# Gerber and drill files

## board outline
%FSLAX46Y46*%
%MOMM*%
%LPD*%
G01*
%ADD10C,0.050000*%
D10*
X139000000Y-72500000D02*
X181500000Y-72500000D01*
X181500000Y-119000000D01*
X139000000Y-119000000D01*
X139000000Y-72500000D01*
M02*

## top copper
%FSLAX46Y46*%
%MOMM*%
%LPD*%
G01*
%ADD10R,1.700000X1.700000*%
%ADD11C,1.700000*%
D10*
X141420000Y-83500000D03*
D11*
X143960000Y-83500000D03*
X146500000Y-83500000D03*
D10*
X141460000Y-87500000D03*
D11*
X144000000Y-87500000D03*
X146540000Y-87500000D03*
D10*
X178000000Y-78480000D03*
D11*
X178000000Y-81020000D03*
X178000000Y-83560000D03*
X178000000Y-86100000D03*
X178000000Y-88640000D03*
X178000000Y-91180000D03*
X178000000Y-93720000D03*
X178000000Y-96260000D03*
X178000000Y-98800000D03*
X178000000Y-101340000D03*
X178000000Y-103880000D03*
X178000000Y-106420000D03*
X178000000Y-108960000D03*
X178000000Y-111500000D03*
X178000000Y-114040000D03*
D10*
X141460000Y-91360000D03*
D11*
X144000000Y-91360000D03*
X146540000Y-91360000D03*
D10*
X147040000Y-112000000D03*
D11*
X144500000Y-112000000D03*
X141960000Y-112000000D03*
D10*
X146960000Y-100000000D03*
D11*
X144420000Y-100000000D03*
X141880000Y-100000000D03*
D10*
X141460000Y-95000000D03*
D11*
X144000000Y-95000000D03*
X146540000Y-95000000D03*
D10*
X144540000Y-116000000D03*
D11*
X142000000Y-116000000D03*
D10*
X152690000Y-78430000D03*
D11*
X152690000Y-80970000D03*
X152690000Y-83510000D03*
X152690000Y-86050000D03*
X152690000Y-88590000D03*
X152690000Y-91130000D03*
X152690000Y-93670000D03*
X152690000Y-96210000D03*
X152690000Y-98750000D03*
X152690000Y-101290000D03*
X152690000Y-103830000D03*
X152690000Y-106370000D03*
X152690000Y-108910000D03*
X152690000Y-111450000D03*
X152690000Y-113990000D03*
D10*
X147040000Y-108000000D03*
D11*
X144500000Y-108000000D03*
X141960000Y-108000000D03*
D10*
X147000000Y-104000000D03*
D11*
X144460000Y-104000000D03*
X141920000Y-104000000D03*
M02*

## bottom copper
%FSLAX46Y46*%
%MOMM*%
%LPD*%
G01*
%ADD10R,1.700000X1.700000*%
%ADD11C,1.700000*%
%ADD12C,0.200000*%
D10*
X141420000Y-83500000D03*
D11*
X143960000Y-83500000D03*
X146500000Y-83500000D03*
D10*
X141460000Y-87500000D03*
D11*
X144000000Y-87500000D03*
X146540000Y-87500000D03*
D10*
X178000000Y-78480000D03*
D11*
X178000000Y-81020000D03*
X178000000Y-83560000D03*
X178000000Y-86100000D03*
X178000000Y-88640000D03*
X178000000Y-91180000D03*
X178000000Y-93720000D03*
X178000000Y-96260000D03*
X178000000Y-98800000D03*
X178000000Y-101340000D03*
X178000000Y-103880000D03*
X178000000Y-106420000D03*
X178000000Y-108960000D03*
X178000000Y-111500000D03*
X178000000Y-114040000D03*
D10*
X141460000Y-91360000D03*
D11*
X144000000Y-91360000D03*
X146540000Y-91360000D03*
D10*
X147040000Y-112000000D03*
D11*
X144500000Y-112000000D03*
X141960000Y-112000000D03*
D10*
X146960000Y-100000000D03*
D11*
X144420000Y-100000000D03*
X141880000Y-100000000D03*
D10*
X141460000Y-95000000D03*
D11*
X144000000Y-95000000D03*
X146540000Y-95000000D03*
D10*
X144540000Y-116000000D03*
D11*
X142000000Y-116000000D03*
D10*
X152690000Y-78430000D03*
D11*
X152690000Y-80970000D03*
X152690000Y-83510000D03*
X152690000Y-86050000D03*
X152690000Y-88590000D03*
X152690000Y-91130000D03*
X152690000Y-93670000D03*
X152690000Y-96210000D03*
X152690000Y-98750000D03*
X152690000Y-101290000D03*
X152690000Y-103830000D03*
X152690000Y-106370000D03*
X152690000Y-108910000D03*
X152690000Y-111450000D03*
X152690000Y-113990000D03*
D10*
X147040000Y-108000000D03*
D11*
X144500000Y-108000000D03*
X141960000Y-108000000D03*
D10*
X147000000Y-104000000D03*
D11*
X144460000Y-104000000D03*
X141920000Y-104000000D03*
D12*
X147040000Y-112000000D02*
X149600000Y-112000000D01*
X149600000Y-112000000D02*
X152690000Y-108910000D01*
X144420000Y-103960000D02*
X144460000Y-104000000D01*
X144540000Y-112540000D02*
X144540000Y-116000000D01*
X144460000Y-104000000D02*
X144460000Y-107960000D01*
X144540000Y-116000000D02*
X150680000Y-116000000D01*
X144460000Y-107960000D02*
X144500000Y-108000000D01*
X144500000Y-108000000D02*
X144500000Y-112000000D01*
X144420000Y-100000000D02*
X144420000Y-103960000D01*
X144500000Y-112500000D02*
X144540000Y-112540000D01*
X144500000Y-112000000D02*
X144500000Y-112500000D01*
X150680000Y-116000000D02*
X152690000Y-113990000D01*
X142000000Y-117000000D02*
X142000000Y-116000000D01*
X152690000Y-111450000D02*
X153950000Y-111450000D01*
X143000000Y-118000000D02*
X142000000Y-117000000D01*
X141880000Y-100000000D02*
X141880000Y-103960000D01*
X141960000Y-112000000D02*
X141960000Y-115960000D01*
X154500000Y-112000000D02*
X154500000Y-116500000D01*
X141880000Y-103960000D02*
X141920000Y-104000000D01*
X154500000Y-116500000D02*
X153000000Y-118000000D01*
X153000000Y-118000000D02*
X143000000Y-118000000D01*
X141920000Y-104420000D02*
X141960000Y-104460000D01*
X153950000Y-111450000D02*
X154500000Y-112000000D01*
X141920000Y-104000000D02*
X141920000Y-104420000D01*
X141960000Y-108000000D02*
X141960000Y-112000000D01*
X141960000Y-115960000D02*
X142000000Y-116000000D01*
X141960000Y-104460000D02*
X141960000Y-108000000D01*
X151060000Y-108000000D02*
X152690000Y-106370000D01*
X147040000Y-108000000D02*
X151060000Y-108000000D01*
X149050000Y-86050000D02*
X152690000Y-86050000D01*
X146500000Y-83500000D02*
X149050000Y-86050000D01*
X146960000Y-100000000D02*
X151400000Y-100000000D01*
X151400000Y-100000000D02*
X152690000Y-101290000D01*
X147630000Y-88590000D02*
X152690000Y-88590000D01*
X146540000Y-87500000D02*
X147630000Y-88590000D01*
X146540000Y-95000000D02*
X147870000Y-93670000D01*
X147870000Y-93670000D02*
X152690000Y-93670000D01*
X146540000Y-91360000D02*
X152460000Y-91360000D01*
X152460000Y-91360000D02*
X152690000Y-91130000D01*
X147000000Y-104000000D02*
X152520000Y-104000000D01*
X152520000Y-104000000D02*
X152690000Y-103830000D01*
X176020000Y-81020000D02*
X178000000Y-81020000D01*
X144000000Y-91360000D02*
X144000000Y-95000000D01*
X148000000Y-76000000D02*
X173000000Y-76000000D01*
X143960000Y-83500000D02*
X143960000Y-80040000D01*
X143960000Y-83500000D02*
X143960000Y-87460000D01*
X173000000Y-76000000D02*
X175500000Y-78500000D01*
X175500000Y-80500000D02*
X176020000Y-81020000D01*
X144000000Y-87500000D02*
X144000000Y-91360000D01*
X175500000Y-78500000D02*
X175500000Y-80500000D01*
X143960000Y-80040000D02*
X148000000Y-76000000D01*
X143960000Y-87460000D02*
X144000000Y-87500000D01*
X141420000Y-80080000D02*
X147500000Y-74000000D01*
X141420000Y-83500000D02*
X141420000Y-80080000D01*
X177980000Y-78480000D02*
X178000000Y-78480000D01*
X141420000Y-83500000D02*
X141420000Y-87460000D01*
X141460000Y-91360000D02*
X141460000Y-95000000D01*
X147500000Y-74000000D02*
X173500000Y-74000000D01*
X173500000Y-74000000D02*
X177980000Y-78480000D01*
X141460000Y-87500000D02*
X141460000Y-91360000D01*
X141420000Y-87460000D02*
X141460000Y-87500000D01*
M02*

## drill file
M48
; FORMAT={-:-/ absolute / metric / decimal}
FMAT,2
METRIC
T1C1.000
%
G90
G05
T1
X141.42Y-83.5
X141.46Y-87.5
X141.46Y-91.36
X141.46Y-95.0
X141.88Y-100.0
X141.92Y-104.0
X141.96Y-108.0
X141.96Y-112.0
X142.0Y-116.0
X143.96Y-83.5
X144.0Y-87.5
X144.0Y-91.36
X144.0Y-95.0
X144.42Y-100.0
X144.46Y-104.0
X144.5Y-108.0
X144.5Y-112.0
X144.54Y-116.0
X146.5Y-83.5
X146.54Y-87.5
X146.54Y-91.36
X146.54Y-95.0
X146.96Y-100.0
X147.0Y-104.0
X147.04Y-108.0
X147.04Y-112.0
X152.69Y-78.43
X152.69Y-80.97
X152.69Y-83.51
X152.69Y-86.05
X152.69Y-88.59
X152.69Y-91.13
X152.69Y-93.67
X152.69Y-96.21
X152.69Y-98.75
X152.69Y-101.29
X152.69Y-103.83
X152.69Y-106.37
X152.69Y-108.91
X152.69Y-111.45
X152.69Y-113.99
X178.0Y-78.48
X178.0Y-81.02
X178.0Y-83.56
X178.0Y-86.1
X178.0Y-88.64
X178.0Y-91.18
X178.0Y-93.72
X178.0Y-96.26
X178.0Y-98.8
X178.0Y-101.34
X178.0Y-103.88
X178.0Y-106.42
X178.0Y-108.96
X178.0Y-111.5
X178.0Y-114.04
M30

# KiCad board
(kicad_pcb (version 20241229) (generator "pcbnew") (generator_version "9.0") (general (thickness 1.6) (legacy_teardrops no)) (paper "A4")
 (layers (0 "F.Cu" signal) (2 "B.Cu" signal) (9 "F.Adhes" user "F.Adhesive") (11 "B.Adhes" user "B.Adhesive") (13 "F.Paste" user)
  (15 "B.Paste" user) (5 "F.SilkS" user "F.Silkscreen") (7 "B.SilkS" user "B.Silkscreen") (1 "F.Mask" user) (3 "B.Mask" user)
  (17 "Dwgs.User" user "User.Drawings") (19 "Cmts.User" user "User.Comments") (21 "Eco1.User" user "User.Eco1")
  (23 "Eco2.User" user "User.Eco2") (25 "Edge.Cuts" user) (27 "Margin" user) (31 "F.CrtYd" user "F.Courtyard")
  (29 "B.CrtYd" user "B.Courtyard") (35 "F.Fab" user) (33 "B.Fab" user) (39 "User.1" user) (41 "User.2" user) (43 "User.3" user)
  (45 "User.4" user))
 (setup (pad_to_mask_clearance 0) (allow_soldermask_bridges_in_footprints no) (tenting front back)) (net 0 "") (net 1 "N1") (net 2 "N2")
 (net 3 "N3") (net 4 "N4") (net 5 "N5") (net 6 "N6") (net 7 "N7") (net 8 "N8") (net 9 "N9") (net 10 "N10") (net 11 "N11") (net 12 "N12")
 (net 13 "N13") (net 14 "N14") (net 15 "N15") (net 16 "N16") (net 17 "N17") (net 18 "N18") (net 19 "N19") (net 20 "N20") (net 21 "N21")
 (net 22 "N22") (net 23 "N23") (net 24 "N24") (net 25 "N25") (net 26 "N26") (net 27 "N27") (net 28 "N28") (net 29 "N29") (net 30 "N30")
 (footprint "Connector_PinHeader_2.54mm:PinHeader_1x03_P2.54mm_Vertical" (layer "F.Cu") (at 141.42 83.5 90)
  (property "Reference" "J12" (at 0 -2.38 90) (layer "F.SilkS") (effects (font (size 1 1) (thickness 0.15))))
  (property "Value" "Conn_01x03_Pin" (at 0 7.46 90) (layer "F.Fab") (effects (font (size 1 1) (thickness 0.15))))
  (pad "1" thru_hole rect (at 0 0 90) (size 1.7 1.7) (drill 1) (layers "*.Cu" "*.Mask") (remove_unused_layers no) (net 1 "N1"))
  (pad "2" thru_hole circle (at 0 2.54 90) (size 1.7 1.7) (drill 1) (layers "*.Cu" "*.Mask") (remove_unused_layers no) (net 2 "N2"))
  (pad "3" thru_hole circle (at 0 5.08 90) (size 1.7 1.7) (drill 1) (layers "*.Cu" "*.Mask") (remove_unused_layers no) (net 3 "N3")))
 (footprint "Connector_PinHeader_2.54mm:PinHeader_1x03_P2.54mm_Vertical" (layer "F.Cu") (at 141.46 87.5 90)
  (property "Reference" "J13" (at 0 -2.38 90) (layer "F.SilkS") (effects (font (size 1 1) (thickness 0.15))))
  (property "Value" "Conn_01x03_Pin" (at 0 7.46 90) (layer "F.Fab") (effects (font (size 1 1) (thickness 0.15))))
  (pad "1" thru_hole rect (at 0 0 90) (size 1.7 1.7) (drill 1) (layers "*.Cu" "*.Mask") (remove_unused_layers no) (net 1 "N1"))
  (pad "2" thru_hole circle (at 0 2.54 90) (size 1.7 1.7) (drill 1) (layers "*.Cu" "*.Mask") (remove_unused_layers no) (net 2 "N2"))
  (pad "3" thru_hole circle (at 0 5.08 90) (size 1.7 1.7) (drill 1) (layers "*.Cu" "*.Mask") (remove_unused_layers no) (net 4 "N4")))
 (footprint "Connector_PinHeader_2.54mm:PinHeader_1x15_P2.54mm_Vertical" (layer "F.Cu") (at 178 78.48)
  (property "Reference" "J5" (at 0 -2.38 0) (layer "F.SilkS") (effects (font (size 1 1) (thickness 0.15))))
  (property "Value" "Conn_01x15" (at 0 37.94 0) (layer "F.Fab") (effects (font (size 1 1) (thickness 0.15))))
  (pad "1" thru_hole rect (at 0 0) (size 1.7 1.7) (drill 1) (layers "*.Cu" "*.Mask") (remove_unused_layers no) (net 1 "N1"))
  (pad "2" thru_hole circle (at 0 2.54) (size 1.7 1.7) (drill 1) (layers "*.Cu" "*.Mask") (remove_unused_layers no) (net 2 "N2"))
  (pad "3" thru_hole circle (at 0 5.08) (size 1.7 1.7) (drill 1) (layers "*.Cu" "*.Mask") (remove_unused_layers no) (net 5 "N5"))
  (pad "4" thru_hole circle (at 0 7.62) (size 1.7 1.7) (drill 1) (layers "*.Cu" "*.Mask") (remove_unused_layers no) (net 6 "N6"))
  (pad "5" thru_hole circle (at 0 10.16) (size 1.7 1.7) (drill 1) (layers "*.Cu" "*.Mask") (remove_unused_layers no) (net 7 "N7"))
  (pad "6" thru_hole circle (at 0 12.7) (size 1.7 1.7) (drill 1) (layers "*.Cu" "*.Mask") (remove_unused_layers no) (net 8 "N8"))
  (pad "7" thru_hole circle (at 0 15.24) (size 1.7 1.7) (drill 1) (layers "*.Cu" "*.Mask") (remove_unused_layers no) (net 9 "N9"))
  (pad "8" thru_hole circle (at 0 17.78) (size 1.7 1.7) (drill 1) (layers "*.Cu" "*.Mask") (remove_unused_layers no) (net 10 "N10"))
  (pad "9" thru_hole circle (at 0 20.32) (size 1.7 1.7) (drill 1) (layers "*.Cu" "*.Mask") (remove_unused_layers no) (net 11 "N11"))
  (pad "10" thru_hole circle (at 0 22.86) (size 1.7 1.7) (drill 1) (layers "*.Cu" "*.Mask") (remove_unused_layers no) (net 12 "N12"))
  (pad "11" thru_hole circle (at 0 25.4) (size 1.7 1.7) (drill 1) (layers "*.Cu" "*.Mask") (remove_unused_layers no) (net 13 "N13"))
  (pad "12" thru_hole circle (at 0 27.94) (size 1.7 1.7) (drill 1) (layers "*.Cu" "*.Mask") (remove_unused_layers no) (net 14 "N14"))
  (pad "13" thru_hole circle (at 0 30.48) (size 1.7 1.7) (drill 1) (layers "*.Cu" "*.Mask") (remove_unused_layers no) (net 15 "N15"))
  (pad "14" thru_hole circle (at 0 33.02) (size 1.7 1.7) (drill 1) (layers "*.Cu" "*.Mask") (remove_unused_layers no) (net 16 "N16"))
  (pad "15" thru_hole circle (at 0 35.56) (size 1.7 1.7) (drill 1) (layers "*.Cu" "*.Mask") (remove_unused_layers no) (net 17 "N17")))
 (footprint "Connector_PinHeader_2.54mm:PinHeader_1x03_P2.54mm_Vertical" (layer "F.Cu") (at 141.46 91.36 90)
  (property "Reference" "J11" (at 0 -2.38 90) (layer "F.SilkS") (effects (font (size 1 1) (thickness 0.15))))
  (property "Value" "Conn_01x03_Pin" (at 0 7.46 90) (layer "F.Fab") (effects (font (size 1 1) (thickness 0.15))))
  (pad "1" thru_hole rect (at 0 0 90) (size 1.7 1.7) (drill 1) (layers "*.Cu" "*.Mask") (remove_unused_layers no) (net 1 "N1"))
  (pad "2" thru_hole circle (at 0 2.54 90) (size 1.7 1.7) (drill 1) (layers "*.Cu" "*.Mask") (remove_unused_layers no) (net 2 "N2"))
  (pad "3" thru_hole circle (at 0 5.08 90) (size 1.7 1.7) (drill 1) (layers "*.Cu" "*.Mask") (remove_unused_layers no) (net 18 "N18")))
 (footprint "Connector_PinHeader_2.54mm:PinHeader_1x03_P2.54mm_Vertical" (layer "F.Cu") (at 147.04 112 -90)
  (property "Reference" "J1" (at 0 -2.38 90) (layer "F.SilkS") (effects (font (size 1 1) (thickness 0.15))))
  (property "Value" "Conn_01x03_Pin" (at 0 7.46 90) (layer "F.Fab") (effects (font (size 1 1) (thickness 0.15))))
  (pad "1" thru_hole rect (at 0 0 270) (size 1.7 1.7) (drill 1) (layers "*.Cu" "*.Mask") (remove_unused_layers no) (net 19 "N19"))
  (pad "2" thru_hole circle (at 0 2.54 270) (size 1.7 1.7) (drill 1) (layers "*.Cu" "*.Mask") (remove_unused_layers no) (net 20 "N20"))
  (pad "3" thru_hole circle (at 0 5.08 270) (size 1.7 1.7) (drill 1) (layers "*.Cu" "*.Mask") (remove_unused_layers no) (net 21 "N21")))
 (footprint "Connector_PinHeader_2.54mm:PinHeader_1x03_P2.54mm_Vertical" (layer "F.Cu") (at 146.96 100 -90)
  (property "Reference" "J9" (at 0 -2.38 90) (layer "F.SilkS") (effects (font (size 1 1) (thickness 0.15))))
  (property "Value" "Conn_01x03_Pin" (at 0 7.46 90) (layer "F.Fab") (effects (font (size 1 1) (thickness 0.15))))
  (pad "1" thru_hole rect (at 0 0 270) (size 1.7 1.7) (drill 1) (layers "*.Cu" "*.Mask") (remove_unused_layers no) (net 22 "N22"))
  (pad "2" thru_hole circle (at 0 2.54 270) (size 1.7 1.7) (drill 1) (layers "*.Cu" "*.Mask") (remove_unused_layers no) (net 20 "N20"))
  (pad "3" thru_hole circle (at 0 5.08 270) (size 1.7 1.7) (drill 1) (layers "*.Cu" "*.Mask") (remove_unused_layers no) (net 21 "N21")))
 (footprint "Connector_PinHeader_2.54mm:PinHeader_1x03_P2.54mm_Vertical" (layer "F.Cu") (at 141.46 95 90)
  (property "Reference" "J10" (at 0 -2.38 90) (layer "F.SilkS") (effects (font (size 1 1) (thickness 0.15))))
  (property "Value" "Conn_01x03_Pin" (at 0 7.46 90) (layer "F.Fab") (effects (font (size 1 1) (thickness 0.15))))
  (pad "1" thru_hole rect (at 0 0 90) (size 1.7 1.7) (drill 1) (layers "*.Cu" "*.Mask") (remove_unused_layers no) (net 1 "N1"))
  (pad "2" thru_hole circle (at 0 2.54 90) (size 1.7 1.7) (drill 1) (layers "*.Cu" "*.Mask") (remove_unused_layers no) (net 2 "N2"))
  (pad "3" thru_hole circle (at 0 5.08 90) (size 1.7 1.7) (drill 1) (layers "*.Cu" "*.Mask") (remove_unused_layers no) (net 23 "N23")))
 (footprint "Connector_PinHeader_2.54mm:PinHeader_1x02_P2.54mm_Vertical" (layer "F.Cu") (at 144.54 116 -90)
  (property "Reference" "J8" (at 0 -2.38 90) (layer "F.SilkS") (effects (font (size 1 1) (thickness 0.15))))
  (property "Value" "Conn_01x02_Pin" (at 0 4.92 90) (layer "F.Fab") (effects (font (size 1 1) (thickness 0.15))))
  (pad "1" thru_hole rect (at 0 0 270) (size 1.7 1.7) (drill 1) (layers "*.Cu" "*.Mask") (remove_unused_layers no) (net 20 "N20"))
  (pad "2" thru_hole circle (at 0 2.54 270) (size 1.7 1.7) (drill 1) (layers "*.Cu" "*.Mask") (remove_unused_layers no) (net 21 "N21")))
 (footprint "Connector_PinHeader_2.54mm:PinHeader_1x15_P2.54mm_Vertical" (layer "F.Cu") (at 152.69 78.43)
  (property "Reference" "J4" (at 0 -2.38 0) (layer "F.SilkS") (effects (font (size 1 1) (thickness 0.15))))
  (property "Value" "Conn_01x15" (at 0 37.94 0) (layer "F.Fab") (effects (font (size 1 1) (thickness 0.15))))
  (pad "1" thru_hole rect (at 0 0) (size 1.7 1.7) (drill 1) (layers "*.Cu" "*.Mask") (remove_unused_layers no) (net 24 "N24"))
  (pad "2" thru_hole circle (at 0 2.54) (size 1.7 1.7) (drill 1) (layers "*.Cu" "*.Mask") (remove_unused_layers no) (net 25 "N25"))
  (pad "3" thru_hole circle (at 0 5.08) (size 1.7 1.7) (drill 1) (layers "*.Cu" "*.Mask") (remove_unused_layers no) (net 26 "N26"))
  (pad "4" thru_hole circle (at 0 7.62) (size 1.7 1.7) (drill 1) (layers "*.Cu" "*.Mask") (remove_unused_layers no) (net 3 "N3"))
  (pad "5" thru_hole circle (at 0 10.16) (size 1.7 1.7) (drill 1) (layers "*.Cu" "*.Mask") (remove_unused_layers no) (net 4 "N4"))
  (pad "6" thru_hole circle (at 0 12.7) (size 1.7 1.7) (drill 1) (layers "*.Cu" "*.Mask") (remove_unused_layers no) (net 18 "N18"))
  (pad "7" thru_hole circle (at 0 15.24) (size 1.7 1.7) (drill 1) (layers "*.Cu" "*.Mask") (remove_unused_layers no) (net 23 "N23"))
  (pad "8" thru_hole circle (at 0 17.78) (size 1.7 1.7) (drill 1) (layers "*.Cu" "*.Mask") (remove_unused_layers no) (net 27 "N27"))
  (pad "9" thru_hole circle (at 0 20.32) (size 1.7 1.7) (drill 1) (layers "*.Cu" "*.Mask") (remove_unused_layers no) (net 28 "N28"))
  (pad "10" thru_hole circle (at 0 22.86) (size 1.7 1.7) (drill 1) (layers "*.Cu" "*.Mask") (remove_unused_layers no) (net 22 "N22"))
  (pad "11" thru_hole circle (at 0 25.4) (size 1.7 1.7) (drill 1) (layers "*.Cu" "*.Mask") (remove_unused_layers no) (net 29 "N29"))
  (pad "12" thru_hole circle (at 0 27.94) (size 1.7 1.7) (drill 1) (layers "*.Cu" "*.Mask") (remove_unused_layers no) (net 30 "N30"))
  (pad "13" thru_hole circle (at 0 30.48) (size 1.7 1.7) (drill 1) (layers "*.Cu" "*.Mask") (remove_unused_layers no) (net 19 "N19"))
  (pad "14" thru_hole circle (at 0 33.02) (size 1.7 1.7) (drill 1) (layers "*.Cu" "*.Mask") (remove_unused_layers no) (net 21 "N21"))
  (pad "15" thru_hole circle (at 0 35.56) (size 1.7 1.7) (drill 1) (layers "*.Cu" "*.Mask") (remove_unused_layers no) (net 20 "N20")))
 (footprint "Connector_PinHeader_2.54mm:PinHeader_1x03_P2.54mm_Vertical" (layer "F.Cu") (at 147.04 108 -90)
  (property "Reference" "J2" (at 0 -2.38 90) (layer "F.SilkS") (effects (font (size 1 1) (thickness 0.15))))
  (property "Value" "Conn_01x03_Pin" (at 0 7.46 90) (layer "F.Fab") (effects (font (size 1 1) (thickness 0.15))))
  (pad "1" thru_hole rect (at 0 0 270) (size 1.7 1.7) (drill 1) (layers "*.Cu" "*.Mask") (remove_unused_layers no) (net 30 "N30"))
  (pad "2" thru_hole circle (at 0 2.54 270) (size 1.7 1.7) (drill 1) (layers "*.Cu" "*.Mask") (remove_unused_layers no) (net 20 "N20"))
  (pad "3" thru_hole circle (at 0 5.08 270) (size 1.7 1.7) (drill 1) (layers "*.Cu" "*.Mask") (remove_unused_layers no) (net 21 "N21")))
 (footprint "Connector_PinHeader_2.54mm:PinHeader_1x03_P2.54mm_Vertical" (layer "F.Cu") (at 147 104 -90)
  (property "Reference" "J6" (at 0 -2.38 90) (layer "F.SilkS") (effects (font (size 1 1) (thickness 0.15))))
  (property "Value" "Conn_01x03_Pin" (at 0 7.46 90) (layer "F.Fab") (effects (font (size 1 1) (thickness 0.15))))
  (pad "1" thru_hole rect (at 0 0 270) (size 1.7 1.7) (drill 1) (layers "*.Cu" "*.Mask") (remove_unused_layers no) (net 29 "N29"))
  (pad "2" thru_hole circle (at 0 2.54 270) (size 1.7 1.7) (drill 1) (layers "*.Cu" "*.Mask") (remove_unused_layers no) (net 20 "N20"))
  (pad "3" thru_hole circle (at 0 5.08 270) (size 1.7 1.7) (drill 1) (layers "*.Cu" "*.Mask") (remove_unused_layers no) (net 21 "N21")))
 (gr_rect (start 139 72.5) (end 181.5 119) (stroke (width 0.05) (type default)) (fill no) (layer "Edge.Cuts"))
 (segment (start 147.04 112) (end 149.6 112) (width 0.2) (layer "B.Cu") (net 19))
 (segment (start 149.6 112) (end 152.69 108.91) (width 0.2) (layer "B.Cu") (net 19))
 (segment (start 144.42 103.96) (end 144.46 104) (width 0.2) (layer "B.Cu") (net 20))
 (segment (start 144.54 112.54) (end 144.54 116) (width 0.2) (layer "B.Cu") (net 20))
 (segment (start 144.46 104) (end 144.46 107.96) (width 0.2) (layer "B.Cu") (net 20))
 (segment (start 144.54 116) (end 150.68 116) (width 0.2) (layer "B.Cu") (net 20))
 (segment (start 144.46 107.96) (end 144.5 108) (width 0.2) (layer "B.Cu") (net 20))
 (segment (start 144.5 108) (end 144.5 112) (width 0.2) (layer "B.Cu") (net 20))
 (segment (start 144.42 100) (end 144.42 103.96) (width 0.2) (layer "B.Cu") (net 20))
 (segment (start 144.5 112.5) (end 144.54 112.54) (width 0.2) (layer "B.Cu") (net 20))
 (segment (start 144.5 112) (end 144.5 112.5) (width 0.2) (layer "B.Cu") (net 20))
 (segment (start 150.68 116) (end 152.69 113.99) (width 0.2) (layer "B.Cu") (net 20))
 (segment (start 142 117) (end 142 116) (width 0.2) (layer "B.Cu") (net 21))
 (segment (start 152.69 111.45) (end 153.95 111.45) (width 0.2) (layer "B.Cu") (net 21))
 (segment (start 143 118) (end 142 117) (width 0.2) (layer "B.Cu") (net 21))
 (segment (start 141.88 100) (end 141.88 103.96) (width 0.2) (layer "B.Cu") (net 21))
 (segment (start 141.96 112) (end 141.96 115.96) (width 0.2) (layer "B.Cu") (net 21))
 (segment (start 154.5 112) (end 154.5 116.5) (width 0.2) (layer "B.Cu") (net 21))
 (segment (start 141.88 103.96) (end 141.92 104) (width 0.2) (layer "B.Cu") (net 21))
 (segment (start 154.5 116.5) (end 153 118) (width 0.2) (layer "B.Cu") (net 21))
 (segment (start 153 118) (end 143 118) (width 0.2) (layer "B.Cu") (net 21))
 (segment (start 141.92 104.42) (end 141.96 104.46) (width 0.2) (layer "B.Cu") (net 21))
 (segment (start 153.95 111.45) (end 154.5 112) (width 0.2) (layer "B.Cu") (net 21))
 (segment (start 141.92 104) (end 141.92 104.42) (width 0.2) (layer "B.Cu") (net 21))
 (segment (start 141.96 108) (end 141.96 112) (width 0.2) (layer "B.Cu") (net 21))
 (segment (start 141.96 115.96) (end 142 116) (width 0.2) (layer "B.Cu") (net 21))
 (segment (start 141.96 104.46) (end 141.96 108) (width 0.2) (layer "B.Cu") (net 21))
 (segment (start 151.06 108) (end 152.69 106.37) (width 0.2) (layer "B.Cu") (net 30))
 (segment (start 147.04 108) (end 151.06 108) (width 0.2) (layer "B.Cu") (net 30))
 (segment (start 149.05 86.05) (end 152.69 86.05) (width 0.2) (layer "B.Cu") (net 3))
 (segment (start 146.5 83.5) (end 149.05 86.05) (width 0.2) (layer "B.Cu") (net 3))
 (segment (start 146.96 100) (end 151.4 100) (width 0.2) (layer "B.Cu") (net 22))
 (segment (start 151.4 100) (end 152.69 101.29) (width 0.2) (layer "B.Cu") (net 22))
 (segment (start 147.63 88.59) (end 152.69 88.59) (width 0.2) (layer "B.Cu") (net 4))
 (segment (start 146.54 87.5) (end 147.63 88.59) (width 0.2) (layer "B.Cu") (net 4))
 (segment (start 146.54 95) (end 147.87 93.67) (width 0.2) (layer "B.Cu") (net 23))
 (segment (start 147.87 93.67) (end 152.69 93.67) (width 0.2) (layer "B.Cu") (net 23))
 (segment (start 146.54 91.36) (end 152.46 91.36) (width 0.2) (layer "B.Cu") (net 18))
 (segment (start 152.46 91.36) (end 152.69 91.13) (width 0.2) (layer "B.Cu") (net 18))
 (segment (start 147 104) (end 152.52 104) (width 0.2) (layer "B.Cu") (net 29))
 (segment (start 152.52 104) (end 152.69 103.83) (width 0.2) (layer "B.Cu") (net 29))
 (segment (start 176.02 81.02) (end 178 81.02) (width 0.2) (layer "B.Cu") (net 2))
 (segment (start 144 91.36) (end 144 95) (width 0.2) (layer "B.Cu") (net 2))
 (segment (start 148 76) (end 173 76) (width 0.2) (layer "B.Cu") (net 2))
 (segment (start 143.96 83.5) (end 143.96 80.04) (width 0.2) (layer "B.Cu") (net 2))
 (segment (start 143.96 83.5) (end 143.96 87.46) (width 0.2) (layer "B.Cu") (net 2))
 (segment (start 173 76) (end 175.5 78.5) (width 0.2) (layer "B.Cu") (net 2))
 (segment (start 175.5 80.5) (end 176.02 81.02) (width 0.2) (layer "B.Cu") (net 2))
 (segment (start 144 87.5) (end 144 91.36) (width 0.2) (layer "B.Cu") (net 2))
 (segment (start 175.5 78.5) (end 175.5 80.5) (width 0.2) (layer "B.Cu") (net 2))
 (segment (start 143.96 80.04) (end 148 76) (width 0.2) (layer "B.Cu") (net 2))
 (segment (start 143.96 87.46) (end 144 87.5) (width 0.2) (layer "B.Cu") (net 2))
 (segment (start 141.42 80.08) (end 147.5 74) (width 0.2) (layer "B.Cu") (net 1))
 (segment (start 141.42 83.5) (end 141.42 80.08) (width 0.2) (layer "B.Cu") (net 1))
 (segment (start 177.98 78.48) (end 178 78.48) (width 0.2) (layer "B.Cu") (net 1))
 (segment (start 141.42 83.5) (end 141.42 87.46) (width 0.2) (layer "B.Cu") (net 1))
 (segment (start 141.46 91.36) (end 141.46 95) (width 0.2) (layer "B.Cu") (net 1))
 (segment (start 147.5 74) (end 173.5 74) (width 0.2) (layer "B.Cu") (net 1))
 (segment (start 173.5 74) (end 177.98 78.48) (width 0.2) (layer "B.Cu") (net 1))
 (segment (start 141.46 87.5) (end 141.46 91.36) (width 0.2) (layer "B.Cu") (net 1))
 (segment (start 141.42 87.46) (end 141.46 87.5) (width 0.2) (layer "B.Cu") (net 1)))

